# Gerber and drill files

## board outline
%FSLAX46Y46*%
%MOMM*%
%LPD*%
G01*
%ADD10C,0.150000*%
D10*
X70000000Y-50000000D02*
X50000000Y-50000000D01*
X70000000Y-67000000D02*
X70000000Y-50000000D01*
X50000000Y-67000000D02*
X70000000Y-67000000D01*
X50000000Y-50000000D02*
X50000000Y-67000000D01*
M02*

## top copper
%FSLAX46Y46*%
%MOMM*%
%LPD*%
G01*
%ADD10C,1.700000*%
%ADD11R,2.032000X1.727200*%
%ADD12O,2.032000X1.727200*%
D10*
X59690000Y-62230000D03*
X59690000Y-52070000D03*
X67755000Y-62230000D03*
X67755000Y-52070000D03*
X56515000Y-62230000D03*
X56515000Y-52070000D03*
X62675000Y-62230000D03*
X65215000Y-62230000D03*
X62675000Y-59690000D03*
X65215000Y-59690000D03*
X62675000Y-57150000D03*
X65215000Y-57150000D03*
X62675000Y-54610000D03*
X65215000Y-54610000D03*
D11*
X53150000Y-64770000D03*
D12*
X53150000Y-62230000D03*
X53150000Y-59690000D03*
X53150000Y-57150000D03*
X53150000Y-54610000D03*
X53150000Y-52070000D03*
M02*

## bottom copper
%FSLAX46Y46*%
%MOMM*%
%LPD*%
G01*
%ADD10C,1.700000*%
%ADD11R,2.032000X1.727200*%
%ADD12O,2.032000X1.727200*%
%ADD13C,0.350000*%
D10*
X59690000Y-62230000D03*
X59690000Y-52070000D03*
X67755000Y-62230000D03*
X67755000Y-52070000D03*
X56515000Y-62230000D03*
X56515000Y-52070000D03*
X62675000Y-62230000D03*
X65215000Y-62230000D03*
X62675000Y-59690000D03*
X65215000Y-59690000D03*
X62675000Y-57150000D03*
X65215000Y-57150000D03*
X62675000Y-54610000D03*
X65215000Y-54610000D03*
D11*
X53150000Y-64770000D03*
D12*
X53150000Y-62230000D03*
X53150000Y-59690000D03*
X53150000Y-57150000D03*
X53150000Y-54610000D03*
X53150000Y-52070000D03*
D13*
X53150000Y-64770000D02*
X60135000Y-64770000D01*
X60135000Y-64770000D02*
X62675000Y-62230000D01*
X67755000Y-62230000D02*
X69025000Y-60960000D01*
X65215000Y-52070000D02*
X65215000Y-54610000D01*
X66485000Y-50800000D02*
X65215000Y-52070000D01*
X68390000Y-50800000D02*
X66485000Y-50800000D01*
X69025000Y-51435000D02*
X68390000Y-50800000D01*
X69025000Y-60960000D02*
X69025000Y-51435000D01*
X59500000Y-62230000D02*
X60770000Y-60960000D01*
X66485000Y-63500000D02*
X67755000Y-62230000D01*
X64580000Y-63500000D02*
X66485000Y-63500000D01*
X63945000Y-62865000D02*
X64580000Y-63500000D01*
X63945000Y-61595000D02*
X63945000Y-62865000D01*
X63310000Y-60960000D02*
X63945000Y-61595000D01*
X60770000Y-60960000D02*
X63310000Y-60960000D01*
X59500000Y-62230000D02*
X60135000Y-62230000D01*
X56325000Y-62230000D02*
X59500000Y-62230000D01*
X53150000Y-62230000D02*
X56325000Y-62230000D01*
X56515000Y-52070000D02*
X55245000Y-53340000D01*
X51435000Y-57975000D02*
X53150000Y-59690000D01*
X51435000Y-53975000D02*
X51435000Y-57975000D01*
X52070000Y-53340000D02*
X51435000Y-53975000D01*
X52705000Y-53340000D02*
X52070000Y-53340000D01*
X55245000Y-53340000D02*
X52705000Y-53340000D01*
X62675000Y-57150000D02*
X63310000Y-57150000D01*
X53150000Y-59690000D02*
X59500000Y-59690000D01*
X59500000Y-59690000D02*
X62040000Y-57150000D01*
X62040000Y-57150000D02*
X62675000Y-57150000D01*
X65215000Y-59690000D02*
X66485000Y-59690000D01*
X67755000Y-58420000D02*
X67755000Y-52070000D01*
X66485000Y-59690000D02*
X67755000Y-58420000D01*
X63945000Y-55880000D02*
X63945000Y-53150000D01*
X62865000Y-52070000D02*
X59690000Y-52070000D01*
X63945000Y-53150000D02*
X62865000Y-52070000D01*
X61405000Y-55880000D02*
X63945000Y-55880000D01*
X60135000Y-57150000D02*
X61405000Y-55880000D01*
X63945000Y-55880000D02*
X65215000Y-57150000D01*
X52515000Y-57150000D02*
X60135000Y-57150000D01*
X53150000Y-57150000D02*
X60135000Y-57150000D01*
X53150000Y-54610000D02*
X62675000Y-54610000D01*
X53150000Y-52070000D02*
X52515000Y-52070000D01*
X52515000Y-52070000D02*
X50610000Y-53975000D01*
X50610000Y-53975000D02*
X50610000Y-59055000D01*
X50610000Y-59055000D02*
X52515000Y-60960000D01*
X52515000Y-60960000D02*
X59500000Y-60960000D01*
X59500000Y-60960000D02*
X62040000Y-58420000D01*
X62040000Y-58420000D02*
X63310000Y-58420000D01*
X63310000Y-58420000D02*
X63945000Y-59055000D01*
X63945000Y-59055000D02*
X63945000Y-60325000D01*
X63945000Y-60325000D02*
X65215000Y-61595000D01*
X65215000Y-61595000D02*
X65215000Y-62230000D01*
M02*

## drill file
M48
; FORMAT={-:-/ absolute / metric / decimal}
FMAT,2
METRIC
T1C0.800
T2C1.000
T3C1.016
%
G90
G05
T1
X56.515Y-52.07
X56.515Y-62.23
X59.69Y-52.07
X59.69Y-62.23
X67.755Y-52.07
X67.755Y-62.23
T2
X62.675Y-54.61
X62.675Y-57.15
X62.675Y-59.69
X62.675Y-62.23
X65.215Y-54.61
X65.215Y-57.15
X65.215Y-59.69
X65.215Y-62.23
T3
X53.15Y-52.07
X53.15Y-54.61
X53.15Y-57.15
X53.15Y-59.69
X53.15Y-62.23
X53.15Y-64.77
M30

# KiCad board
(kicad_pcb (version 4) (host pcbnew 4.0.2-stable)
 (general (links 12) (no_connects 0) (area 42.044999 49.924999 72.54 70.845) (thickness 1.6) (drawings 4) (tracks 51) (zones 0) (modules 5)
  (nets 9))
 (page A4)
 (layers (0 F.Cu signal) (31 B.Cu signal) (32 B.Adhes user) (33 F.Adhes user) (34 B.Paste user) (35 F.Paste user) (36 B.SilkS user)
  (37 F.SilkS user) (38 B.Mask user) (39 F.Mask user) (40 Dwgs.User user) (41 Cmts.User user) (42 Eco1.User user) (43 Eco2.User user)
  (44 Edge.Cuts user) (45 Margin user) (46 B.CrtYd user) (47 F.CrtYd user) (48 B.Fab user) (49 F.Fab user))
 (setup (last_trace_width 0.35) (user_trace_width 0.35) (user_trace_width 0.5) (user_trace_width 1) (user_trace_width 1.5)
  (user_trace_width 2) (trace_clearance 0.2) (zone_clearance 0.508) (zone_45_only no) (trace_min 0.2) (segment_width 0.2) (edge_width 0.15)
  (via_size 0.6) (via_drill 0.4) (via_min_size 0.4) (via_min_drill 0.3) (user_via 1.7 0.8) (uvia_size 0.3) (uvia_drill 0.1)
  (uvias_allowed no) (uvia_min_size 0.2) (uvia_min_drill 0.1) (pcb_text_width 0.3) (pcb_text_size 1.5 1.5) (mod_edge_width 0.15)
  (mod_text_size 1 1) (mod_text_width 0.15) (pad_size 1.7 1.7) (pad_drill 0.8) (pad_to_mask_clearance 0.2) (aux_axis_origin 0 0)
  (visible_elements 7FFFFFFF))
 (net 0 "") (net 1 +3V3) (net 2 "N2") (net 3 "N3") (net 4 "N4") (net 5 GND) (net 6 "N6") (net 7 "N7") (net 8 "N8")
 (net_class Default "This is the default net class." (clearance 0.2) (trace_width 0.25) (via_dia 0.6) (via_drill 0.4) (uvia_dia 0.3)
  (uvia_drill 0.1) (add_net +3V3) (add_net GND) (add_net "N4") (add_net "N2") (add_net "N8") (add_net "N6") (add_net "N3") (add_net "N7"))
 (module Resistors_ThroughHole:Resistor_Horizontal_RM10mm (layer F.Cu) (at 59.69 62.23 90)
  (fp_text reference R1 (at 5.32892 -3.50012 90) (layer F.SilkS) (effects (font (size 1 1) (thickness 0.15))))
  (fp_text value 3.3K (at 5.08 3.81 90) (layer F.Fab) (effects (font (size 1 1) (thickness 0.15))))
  (pad 1 thru_hole circle (at 0 0 90) (size 1.7 1.7) (drill 0.8) (layers *.Cu *.SilkS *.Mask) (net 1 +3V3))
  (pad 2 thru_hole circle (at 10.16 0 90) (size 1.7 1.7) (drill 0.8) (layers *.Cu *.SilkS *.Mask) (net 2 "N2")))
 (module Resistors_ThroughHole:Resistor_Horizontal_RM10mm (layer F.Cu) (at 67.755 62.23 90)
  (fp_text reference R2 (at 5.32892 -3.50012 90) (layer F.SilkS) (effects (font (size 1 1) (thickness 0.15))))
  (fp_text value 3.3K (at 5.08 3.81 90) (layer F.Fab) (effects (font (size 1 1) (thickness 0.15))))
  (pad 1 thru_hole circle (at 0 0 90) (size 1.7 1.7) (drill 0.8) (layers *.Cu *.SilkS *.Mask) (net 1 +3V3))
  (pad 2 thru_hole circle (at 10.16 0 90) (size 1.7 1.7) (drill 0.8) (layers *.Cu *.SilkS *.Mask) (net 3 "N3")))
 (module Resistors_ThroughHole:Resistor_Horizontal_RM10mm (layer F.Cu) (at 56.515 62.23 90)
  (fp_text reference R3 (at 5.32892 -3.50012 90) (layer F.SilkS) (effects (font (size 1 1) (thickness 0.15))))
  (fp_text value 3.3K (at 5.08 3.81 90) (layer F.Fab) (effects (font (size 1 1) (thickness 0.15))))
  (pad 1 thru_hole circle (at 0 0 90) (size 1.7 1.7) (drill 0.8) (layers *.Cu *.SilkS *.Mask) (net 1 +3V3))
  (pad 2 thru_hole circle (at 10.16 0 90) (size 1.7 1.7) (drill 0.8) (layers *.Cu *.SilkS *.Mask) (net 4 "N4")))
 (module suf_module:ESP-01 (layer F.Cu) (at 67.12 58.42 180)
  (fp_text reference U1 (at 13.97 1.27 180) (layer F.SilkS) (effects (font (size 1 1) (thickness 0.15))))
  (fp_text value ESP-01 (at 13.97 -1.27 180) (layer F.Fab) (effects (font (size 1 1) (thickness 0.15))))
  (pad 1 thru_hole circle (at 4.445 -3.81 180) (size 1.7 1.7) (drill 1) (layers *.Cu *.Mask F.SilkS) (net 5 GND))
  (pad 2 thru_hole circle (at 1.905 -3.81 180) (size 1.7 1.7) (drill 1) (layers *.Cu *.Mask F.SilkS) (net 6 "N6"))
  (pad 3 thru_hole circle (at 4.445 -1.27 180) (size 1.7 1.7) (drill 1) (layers *.Cu *.Mask F.SilkS) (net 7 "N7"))
  (pad 4 thru_hole circle (at 1.905 -1.27 180) (size 1.7 1.7) (drill 1) (layers *.Cu *.Mask F.SilkS) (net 3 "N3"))
  (pad 5 thru_hole circle (at 4.445 1.27 180) (size 1.7 1.7) (drill 1) (layers *.Cu *.Mask F.SilkS) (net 4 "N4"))
  (pad 6 thru_hole circle (at 1.905 1.27 180) (size 1.7 1.7) (drill 1) (layers *.Cu *.Mask F.SilkS) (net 2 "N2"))
  (pad 7 thru_hole circle (at 4.445 3.81 180) (size 1.7 1.7) (drill 1) (layers *.Cu *.Mask F.SilkS) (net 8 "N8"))
  (pad 8 thru_hole circle (at 1.905 3.81 180) (size 1.7 1.7) (drill 1) (layers *.Cu *.Mask F.SilkS) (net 1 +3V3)))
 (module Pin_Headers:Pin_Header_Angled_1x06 (layer F.Cu) (at 53.15 64.77 180)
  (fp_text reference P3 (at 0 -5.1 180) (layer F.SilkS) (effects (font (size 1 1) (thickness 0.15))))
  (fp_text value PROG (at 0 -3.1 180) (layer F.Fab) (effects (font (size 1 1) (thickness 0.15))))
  (pad 1 thru_hole rect (at 0 0 180) (size 2.032 1.7272) (drill 1.016) (layers *.Cu *.Mask F.SilkS) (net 5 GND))
  (pad 2 thru_hole oval (at 0 2.54 180) (size 2.032 1.7272) (drill 1.016) (layers *.Cu *.Mask F.SilkS) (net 1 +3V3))
  (pad 3 thru_hole oval (at 0 5.08 180) (size 2.032 1.7272) (drill 1.016) (layers *.Cu *.Mask F.SilkS) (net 4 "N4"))
  (pad 4 thru_hole oval (at 0 7.62 180) (size 2.032 1.7272) (drill 1.016) (layers *.Cu *.Mask F.SilkS) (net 2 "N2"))
  (pad 5 thru_hole oval (at 0 10.16 180) (size 2.032 1.7272) (drill 1.016) (layers *.Cu *.Mask F.SilkS) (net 8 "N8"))
  (pad 6 thru_hole oval (at 0 12.7 180) (size 2.032 1.7272) (drill 1.016) (layers *.Cu *.Mask F.SilkS) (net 6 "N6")))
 (gr_line (start 70 50) (end 50 50) (angle 90) (layer Edge.Cuts) (width 0.15))
 (gr_line (start 70 67) (end 70 50) (angle 90) (layer Edge.Cuts) (width 0.15))
 (gr_line (start 50 67) (end 70 67) (angle 90) (layer Edge.Cuts) (width 0.15))
 (gr_line (start 50 50) (end 50 67) (angle 90) (layer Edge.Cuts) (width 0.15))
 (segment (start 53.15 64.77) (end 60.135 64.77) (width 0.35) (layer B.Cu) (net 5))
 (segment (start 60.135 64.77) (end 62.675 62.23) (width 0.35) (layer B.Cu) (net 5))
 (segment (start 67.755 62.23) (end 69.025 60.96) (width 0.35) (layer B.Cu) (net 1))
 (segment (start 65.215 52.07) (end 65.215 54.61) (width 0.35) (layer B.Cu) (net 1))
 (segment (start 66.485 50.8) (end 65.215 52.07) (width 0.35) (layer B.Cu) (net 1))
 (segment (start 68.39 50.8) (end 66.485 50.8) (width 0.35) (layer B.Cu) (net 1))
 (segment (start 69.025 51.435) (end 68.39 50.8) (width 0.35) (layer B.Cu) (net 1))
 (segment (start 69.025 60.96) (end 69.025 51.435) (width 0.35) (layer B.Cu) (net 1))
 (segment (start 59.5 62.23) (end 60.77 60.96) (width 0.35) (layer B.Cu) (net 1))
 (segment (start 66.485 63.5) (end 67.755 62.23) (width 0.35) (layer B.Cu) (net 1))
 (segment (start 64.58 63.5) (end 66.485 63.5) (width 0.35) (layer B.Cu) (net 1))
 (segment (start 63.945 62.865) (end 64.58 63.5) (width 0.35) (layer B.Cu) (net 1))
 (segment (start 63.945 61.595) (end 63.945 62.865) (width 0.35) (layer B.Cu) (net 1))
 (segment (start 63.31 60.96) (end 63.945 61.595) (width 0.35) (layer B.Cu) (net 1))
 (segment (start 60.77 60.96) (end 63.31 60.96) (width 0.35) (layer B.Cu) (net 1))
 (segment (start 59.5 62.23) (end 60.135 62.23) (width 0.35) (layer B.Cu) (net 1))
 (segment (start 56.325 62.23) (end 59.5 62.23) (width 0.35) (layer B.Cu) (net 1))
 (segment (start 53.15 62.23) (end 56.325 62.23) (width 0.35) (layer B.Cu) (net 1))
 (segment (start 56.515 52.07) (end 55.245 53.34) (width 0.35) (layer B.Cu) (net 4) (status 400000))
 (segment (start 51.435 57.975) (end 53.15 59.69) (width 0.35) (layer B.Cu) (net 4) (status 800000))
 (segment (start 51.435 53.975) (end 51.435 57.975) (width 0.35) (layer B.Cu) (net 4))
 (segment (start 52.07 53.34) (end 51.435 53.975) (width 0.35) (layer B.Cu) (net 4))
 (segment (start 52.705 53.34) (end 52.07 53.34) (width 0.35) (layer B.Cu) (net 4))
 (segment (start 55.245 53.34) (end 52.705 53.34) (width 0.35) (layer B.Cu) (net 4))
 (segment (start 62.675 57.15) (end 63.31 57.15) (width 0.35) (layer B.Cu) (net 4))
 (segment (start 53.15 59.69) (end 59.5 59.69) (width 0.35) (layer B.Cu) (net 4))
 (segment (start 59.5 59.69) (end 62.04 57.15) (width 0.35) (layer B.Cu) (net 4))
 (segment (start 62.04 57.15) (end 62.675 57.15) (width 0.35) (layer B.Cu) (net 4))
 (segment (start 65.215 59.69) (end 66.485 59.69) (width 0.35) (layer B.Cu) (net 3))
 (segment (start 67.755 58.42) (end 67.755 52.07) (width 0.35) (layer B.Cu) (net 3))
 (segment (start 66.485 59.69) (end 67.755 58.42) (width 0.35) (layer B.Cu) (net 3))
 (segment (start 63.945 55.88) (end 63.945 53.15) (width 0.35) (layer B.Cu) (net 2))
 (segment (start 62.865 52.07) (end 59.69 52.07) (width 0.35) (layer B.Cu) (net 2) (status 800000))
 (segment (start 63.945 53.15) (end 62.865 52.07) (width 0.35) (layer B.Cu) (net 2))
 (segment (start 61.405 55.88) (end 63.945 55.88) (width 0.35) (layer B.Cu) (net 2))
 (segment (start 60.135 57.15) (end 61.405 55.88) (width 0.35) (layer B.Cu) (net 2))
 (segment (start 63.945 55.88) (end 65.215 57.15) (width 0.35) (layer B.Cu) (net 2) (status 800000))
 (segment (start 52.515 57.15) (end 60.135 57.15) (width 0.35) (layer B.Cu) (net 2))
 (segment (start 53.15 57.15) (end 60.135 57.15) (width 0.35) (layer B.Cu) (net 2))
 (segment (start 53.15 54.61) (end 62.675 54.61) (width 0.35) (layer B.Cu) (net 8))
 (segment (start 53.15 52.07) (end 52.515 52.07) (width 0.35) (layer B.Cu) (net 6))
 (segment (start 52.515 52.07) (end 50.61 53.975) (width 0.35) (layer B.Cu) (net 6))
 (segment (start 50.61 53.975) (end 50.61 59.055) (width 0.35) (layer B.Cu) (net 6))
 (segment (start 50.61 59.055) (end 52.515 60.96) (width 0.35) (layer B.Cu) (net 6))
 (segment (start 52.515 60.96) (end 59.5 60.96) (width 0.35) (layer B.Cu) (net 6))
 (segment (start 59.5 60.96) (end 62.04 58.42) (width 0.35) (layer B.Cu) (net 6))
 (segment (start 62.04 58.42) (end 63.31 58.42) (width 0.35) (layer B.Cu) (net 6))
 (segment (start 63.31 58.42) (end 63.945 59.055) (width 0.35) (layer B.Cu) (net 6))
 (segment (start 63.945 59.055) (end 63.945 60.325) (width 0.35) (layer B.Cu) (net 6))
 (segment (start 63.945 60.325) (end 65.215 61.595) (width 0.35) (layer B.Cu) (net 6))
 (segment (start 65.215 61.595) (end 65.215 62.23) (width 0.35) (layer B.Cu) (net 6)))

